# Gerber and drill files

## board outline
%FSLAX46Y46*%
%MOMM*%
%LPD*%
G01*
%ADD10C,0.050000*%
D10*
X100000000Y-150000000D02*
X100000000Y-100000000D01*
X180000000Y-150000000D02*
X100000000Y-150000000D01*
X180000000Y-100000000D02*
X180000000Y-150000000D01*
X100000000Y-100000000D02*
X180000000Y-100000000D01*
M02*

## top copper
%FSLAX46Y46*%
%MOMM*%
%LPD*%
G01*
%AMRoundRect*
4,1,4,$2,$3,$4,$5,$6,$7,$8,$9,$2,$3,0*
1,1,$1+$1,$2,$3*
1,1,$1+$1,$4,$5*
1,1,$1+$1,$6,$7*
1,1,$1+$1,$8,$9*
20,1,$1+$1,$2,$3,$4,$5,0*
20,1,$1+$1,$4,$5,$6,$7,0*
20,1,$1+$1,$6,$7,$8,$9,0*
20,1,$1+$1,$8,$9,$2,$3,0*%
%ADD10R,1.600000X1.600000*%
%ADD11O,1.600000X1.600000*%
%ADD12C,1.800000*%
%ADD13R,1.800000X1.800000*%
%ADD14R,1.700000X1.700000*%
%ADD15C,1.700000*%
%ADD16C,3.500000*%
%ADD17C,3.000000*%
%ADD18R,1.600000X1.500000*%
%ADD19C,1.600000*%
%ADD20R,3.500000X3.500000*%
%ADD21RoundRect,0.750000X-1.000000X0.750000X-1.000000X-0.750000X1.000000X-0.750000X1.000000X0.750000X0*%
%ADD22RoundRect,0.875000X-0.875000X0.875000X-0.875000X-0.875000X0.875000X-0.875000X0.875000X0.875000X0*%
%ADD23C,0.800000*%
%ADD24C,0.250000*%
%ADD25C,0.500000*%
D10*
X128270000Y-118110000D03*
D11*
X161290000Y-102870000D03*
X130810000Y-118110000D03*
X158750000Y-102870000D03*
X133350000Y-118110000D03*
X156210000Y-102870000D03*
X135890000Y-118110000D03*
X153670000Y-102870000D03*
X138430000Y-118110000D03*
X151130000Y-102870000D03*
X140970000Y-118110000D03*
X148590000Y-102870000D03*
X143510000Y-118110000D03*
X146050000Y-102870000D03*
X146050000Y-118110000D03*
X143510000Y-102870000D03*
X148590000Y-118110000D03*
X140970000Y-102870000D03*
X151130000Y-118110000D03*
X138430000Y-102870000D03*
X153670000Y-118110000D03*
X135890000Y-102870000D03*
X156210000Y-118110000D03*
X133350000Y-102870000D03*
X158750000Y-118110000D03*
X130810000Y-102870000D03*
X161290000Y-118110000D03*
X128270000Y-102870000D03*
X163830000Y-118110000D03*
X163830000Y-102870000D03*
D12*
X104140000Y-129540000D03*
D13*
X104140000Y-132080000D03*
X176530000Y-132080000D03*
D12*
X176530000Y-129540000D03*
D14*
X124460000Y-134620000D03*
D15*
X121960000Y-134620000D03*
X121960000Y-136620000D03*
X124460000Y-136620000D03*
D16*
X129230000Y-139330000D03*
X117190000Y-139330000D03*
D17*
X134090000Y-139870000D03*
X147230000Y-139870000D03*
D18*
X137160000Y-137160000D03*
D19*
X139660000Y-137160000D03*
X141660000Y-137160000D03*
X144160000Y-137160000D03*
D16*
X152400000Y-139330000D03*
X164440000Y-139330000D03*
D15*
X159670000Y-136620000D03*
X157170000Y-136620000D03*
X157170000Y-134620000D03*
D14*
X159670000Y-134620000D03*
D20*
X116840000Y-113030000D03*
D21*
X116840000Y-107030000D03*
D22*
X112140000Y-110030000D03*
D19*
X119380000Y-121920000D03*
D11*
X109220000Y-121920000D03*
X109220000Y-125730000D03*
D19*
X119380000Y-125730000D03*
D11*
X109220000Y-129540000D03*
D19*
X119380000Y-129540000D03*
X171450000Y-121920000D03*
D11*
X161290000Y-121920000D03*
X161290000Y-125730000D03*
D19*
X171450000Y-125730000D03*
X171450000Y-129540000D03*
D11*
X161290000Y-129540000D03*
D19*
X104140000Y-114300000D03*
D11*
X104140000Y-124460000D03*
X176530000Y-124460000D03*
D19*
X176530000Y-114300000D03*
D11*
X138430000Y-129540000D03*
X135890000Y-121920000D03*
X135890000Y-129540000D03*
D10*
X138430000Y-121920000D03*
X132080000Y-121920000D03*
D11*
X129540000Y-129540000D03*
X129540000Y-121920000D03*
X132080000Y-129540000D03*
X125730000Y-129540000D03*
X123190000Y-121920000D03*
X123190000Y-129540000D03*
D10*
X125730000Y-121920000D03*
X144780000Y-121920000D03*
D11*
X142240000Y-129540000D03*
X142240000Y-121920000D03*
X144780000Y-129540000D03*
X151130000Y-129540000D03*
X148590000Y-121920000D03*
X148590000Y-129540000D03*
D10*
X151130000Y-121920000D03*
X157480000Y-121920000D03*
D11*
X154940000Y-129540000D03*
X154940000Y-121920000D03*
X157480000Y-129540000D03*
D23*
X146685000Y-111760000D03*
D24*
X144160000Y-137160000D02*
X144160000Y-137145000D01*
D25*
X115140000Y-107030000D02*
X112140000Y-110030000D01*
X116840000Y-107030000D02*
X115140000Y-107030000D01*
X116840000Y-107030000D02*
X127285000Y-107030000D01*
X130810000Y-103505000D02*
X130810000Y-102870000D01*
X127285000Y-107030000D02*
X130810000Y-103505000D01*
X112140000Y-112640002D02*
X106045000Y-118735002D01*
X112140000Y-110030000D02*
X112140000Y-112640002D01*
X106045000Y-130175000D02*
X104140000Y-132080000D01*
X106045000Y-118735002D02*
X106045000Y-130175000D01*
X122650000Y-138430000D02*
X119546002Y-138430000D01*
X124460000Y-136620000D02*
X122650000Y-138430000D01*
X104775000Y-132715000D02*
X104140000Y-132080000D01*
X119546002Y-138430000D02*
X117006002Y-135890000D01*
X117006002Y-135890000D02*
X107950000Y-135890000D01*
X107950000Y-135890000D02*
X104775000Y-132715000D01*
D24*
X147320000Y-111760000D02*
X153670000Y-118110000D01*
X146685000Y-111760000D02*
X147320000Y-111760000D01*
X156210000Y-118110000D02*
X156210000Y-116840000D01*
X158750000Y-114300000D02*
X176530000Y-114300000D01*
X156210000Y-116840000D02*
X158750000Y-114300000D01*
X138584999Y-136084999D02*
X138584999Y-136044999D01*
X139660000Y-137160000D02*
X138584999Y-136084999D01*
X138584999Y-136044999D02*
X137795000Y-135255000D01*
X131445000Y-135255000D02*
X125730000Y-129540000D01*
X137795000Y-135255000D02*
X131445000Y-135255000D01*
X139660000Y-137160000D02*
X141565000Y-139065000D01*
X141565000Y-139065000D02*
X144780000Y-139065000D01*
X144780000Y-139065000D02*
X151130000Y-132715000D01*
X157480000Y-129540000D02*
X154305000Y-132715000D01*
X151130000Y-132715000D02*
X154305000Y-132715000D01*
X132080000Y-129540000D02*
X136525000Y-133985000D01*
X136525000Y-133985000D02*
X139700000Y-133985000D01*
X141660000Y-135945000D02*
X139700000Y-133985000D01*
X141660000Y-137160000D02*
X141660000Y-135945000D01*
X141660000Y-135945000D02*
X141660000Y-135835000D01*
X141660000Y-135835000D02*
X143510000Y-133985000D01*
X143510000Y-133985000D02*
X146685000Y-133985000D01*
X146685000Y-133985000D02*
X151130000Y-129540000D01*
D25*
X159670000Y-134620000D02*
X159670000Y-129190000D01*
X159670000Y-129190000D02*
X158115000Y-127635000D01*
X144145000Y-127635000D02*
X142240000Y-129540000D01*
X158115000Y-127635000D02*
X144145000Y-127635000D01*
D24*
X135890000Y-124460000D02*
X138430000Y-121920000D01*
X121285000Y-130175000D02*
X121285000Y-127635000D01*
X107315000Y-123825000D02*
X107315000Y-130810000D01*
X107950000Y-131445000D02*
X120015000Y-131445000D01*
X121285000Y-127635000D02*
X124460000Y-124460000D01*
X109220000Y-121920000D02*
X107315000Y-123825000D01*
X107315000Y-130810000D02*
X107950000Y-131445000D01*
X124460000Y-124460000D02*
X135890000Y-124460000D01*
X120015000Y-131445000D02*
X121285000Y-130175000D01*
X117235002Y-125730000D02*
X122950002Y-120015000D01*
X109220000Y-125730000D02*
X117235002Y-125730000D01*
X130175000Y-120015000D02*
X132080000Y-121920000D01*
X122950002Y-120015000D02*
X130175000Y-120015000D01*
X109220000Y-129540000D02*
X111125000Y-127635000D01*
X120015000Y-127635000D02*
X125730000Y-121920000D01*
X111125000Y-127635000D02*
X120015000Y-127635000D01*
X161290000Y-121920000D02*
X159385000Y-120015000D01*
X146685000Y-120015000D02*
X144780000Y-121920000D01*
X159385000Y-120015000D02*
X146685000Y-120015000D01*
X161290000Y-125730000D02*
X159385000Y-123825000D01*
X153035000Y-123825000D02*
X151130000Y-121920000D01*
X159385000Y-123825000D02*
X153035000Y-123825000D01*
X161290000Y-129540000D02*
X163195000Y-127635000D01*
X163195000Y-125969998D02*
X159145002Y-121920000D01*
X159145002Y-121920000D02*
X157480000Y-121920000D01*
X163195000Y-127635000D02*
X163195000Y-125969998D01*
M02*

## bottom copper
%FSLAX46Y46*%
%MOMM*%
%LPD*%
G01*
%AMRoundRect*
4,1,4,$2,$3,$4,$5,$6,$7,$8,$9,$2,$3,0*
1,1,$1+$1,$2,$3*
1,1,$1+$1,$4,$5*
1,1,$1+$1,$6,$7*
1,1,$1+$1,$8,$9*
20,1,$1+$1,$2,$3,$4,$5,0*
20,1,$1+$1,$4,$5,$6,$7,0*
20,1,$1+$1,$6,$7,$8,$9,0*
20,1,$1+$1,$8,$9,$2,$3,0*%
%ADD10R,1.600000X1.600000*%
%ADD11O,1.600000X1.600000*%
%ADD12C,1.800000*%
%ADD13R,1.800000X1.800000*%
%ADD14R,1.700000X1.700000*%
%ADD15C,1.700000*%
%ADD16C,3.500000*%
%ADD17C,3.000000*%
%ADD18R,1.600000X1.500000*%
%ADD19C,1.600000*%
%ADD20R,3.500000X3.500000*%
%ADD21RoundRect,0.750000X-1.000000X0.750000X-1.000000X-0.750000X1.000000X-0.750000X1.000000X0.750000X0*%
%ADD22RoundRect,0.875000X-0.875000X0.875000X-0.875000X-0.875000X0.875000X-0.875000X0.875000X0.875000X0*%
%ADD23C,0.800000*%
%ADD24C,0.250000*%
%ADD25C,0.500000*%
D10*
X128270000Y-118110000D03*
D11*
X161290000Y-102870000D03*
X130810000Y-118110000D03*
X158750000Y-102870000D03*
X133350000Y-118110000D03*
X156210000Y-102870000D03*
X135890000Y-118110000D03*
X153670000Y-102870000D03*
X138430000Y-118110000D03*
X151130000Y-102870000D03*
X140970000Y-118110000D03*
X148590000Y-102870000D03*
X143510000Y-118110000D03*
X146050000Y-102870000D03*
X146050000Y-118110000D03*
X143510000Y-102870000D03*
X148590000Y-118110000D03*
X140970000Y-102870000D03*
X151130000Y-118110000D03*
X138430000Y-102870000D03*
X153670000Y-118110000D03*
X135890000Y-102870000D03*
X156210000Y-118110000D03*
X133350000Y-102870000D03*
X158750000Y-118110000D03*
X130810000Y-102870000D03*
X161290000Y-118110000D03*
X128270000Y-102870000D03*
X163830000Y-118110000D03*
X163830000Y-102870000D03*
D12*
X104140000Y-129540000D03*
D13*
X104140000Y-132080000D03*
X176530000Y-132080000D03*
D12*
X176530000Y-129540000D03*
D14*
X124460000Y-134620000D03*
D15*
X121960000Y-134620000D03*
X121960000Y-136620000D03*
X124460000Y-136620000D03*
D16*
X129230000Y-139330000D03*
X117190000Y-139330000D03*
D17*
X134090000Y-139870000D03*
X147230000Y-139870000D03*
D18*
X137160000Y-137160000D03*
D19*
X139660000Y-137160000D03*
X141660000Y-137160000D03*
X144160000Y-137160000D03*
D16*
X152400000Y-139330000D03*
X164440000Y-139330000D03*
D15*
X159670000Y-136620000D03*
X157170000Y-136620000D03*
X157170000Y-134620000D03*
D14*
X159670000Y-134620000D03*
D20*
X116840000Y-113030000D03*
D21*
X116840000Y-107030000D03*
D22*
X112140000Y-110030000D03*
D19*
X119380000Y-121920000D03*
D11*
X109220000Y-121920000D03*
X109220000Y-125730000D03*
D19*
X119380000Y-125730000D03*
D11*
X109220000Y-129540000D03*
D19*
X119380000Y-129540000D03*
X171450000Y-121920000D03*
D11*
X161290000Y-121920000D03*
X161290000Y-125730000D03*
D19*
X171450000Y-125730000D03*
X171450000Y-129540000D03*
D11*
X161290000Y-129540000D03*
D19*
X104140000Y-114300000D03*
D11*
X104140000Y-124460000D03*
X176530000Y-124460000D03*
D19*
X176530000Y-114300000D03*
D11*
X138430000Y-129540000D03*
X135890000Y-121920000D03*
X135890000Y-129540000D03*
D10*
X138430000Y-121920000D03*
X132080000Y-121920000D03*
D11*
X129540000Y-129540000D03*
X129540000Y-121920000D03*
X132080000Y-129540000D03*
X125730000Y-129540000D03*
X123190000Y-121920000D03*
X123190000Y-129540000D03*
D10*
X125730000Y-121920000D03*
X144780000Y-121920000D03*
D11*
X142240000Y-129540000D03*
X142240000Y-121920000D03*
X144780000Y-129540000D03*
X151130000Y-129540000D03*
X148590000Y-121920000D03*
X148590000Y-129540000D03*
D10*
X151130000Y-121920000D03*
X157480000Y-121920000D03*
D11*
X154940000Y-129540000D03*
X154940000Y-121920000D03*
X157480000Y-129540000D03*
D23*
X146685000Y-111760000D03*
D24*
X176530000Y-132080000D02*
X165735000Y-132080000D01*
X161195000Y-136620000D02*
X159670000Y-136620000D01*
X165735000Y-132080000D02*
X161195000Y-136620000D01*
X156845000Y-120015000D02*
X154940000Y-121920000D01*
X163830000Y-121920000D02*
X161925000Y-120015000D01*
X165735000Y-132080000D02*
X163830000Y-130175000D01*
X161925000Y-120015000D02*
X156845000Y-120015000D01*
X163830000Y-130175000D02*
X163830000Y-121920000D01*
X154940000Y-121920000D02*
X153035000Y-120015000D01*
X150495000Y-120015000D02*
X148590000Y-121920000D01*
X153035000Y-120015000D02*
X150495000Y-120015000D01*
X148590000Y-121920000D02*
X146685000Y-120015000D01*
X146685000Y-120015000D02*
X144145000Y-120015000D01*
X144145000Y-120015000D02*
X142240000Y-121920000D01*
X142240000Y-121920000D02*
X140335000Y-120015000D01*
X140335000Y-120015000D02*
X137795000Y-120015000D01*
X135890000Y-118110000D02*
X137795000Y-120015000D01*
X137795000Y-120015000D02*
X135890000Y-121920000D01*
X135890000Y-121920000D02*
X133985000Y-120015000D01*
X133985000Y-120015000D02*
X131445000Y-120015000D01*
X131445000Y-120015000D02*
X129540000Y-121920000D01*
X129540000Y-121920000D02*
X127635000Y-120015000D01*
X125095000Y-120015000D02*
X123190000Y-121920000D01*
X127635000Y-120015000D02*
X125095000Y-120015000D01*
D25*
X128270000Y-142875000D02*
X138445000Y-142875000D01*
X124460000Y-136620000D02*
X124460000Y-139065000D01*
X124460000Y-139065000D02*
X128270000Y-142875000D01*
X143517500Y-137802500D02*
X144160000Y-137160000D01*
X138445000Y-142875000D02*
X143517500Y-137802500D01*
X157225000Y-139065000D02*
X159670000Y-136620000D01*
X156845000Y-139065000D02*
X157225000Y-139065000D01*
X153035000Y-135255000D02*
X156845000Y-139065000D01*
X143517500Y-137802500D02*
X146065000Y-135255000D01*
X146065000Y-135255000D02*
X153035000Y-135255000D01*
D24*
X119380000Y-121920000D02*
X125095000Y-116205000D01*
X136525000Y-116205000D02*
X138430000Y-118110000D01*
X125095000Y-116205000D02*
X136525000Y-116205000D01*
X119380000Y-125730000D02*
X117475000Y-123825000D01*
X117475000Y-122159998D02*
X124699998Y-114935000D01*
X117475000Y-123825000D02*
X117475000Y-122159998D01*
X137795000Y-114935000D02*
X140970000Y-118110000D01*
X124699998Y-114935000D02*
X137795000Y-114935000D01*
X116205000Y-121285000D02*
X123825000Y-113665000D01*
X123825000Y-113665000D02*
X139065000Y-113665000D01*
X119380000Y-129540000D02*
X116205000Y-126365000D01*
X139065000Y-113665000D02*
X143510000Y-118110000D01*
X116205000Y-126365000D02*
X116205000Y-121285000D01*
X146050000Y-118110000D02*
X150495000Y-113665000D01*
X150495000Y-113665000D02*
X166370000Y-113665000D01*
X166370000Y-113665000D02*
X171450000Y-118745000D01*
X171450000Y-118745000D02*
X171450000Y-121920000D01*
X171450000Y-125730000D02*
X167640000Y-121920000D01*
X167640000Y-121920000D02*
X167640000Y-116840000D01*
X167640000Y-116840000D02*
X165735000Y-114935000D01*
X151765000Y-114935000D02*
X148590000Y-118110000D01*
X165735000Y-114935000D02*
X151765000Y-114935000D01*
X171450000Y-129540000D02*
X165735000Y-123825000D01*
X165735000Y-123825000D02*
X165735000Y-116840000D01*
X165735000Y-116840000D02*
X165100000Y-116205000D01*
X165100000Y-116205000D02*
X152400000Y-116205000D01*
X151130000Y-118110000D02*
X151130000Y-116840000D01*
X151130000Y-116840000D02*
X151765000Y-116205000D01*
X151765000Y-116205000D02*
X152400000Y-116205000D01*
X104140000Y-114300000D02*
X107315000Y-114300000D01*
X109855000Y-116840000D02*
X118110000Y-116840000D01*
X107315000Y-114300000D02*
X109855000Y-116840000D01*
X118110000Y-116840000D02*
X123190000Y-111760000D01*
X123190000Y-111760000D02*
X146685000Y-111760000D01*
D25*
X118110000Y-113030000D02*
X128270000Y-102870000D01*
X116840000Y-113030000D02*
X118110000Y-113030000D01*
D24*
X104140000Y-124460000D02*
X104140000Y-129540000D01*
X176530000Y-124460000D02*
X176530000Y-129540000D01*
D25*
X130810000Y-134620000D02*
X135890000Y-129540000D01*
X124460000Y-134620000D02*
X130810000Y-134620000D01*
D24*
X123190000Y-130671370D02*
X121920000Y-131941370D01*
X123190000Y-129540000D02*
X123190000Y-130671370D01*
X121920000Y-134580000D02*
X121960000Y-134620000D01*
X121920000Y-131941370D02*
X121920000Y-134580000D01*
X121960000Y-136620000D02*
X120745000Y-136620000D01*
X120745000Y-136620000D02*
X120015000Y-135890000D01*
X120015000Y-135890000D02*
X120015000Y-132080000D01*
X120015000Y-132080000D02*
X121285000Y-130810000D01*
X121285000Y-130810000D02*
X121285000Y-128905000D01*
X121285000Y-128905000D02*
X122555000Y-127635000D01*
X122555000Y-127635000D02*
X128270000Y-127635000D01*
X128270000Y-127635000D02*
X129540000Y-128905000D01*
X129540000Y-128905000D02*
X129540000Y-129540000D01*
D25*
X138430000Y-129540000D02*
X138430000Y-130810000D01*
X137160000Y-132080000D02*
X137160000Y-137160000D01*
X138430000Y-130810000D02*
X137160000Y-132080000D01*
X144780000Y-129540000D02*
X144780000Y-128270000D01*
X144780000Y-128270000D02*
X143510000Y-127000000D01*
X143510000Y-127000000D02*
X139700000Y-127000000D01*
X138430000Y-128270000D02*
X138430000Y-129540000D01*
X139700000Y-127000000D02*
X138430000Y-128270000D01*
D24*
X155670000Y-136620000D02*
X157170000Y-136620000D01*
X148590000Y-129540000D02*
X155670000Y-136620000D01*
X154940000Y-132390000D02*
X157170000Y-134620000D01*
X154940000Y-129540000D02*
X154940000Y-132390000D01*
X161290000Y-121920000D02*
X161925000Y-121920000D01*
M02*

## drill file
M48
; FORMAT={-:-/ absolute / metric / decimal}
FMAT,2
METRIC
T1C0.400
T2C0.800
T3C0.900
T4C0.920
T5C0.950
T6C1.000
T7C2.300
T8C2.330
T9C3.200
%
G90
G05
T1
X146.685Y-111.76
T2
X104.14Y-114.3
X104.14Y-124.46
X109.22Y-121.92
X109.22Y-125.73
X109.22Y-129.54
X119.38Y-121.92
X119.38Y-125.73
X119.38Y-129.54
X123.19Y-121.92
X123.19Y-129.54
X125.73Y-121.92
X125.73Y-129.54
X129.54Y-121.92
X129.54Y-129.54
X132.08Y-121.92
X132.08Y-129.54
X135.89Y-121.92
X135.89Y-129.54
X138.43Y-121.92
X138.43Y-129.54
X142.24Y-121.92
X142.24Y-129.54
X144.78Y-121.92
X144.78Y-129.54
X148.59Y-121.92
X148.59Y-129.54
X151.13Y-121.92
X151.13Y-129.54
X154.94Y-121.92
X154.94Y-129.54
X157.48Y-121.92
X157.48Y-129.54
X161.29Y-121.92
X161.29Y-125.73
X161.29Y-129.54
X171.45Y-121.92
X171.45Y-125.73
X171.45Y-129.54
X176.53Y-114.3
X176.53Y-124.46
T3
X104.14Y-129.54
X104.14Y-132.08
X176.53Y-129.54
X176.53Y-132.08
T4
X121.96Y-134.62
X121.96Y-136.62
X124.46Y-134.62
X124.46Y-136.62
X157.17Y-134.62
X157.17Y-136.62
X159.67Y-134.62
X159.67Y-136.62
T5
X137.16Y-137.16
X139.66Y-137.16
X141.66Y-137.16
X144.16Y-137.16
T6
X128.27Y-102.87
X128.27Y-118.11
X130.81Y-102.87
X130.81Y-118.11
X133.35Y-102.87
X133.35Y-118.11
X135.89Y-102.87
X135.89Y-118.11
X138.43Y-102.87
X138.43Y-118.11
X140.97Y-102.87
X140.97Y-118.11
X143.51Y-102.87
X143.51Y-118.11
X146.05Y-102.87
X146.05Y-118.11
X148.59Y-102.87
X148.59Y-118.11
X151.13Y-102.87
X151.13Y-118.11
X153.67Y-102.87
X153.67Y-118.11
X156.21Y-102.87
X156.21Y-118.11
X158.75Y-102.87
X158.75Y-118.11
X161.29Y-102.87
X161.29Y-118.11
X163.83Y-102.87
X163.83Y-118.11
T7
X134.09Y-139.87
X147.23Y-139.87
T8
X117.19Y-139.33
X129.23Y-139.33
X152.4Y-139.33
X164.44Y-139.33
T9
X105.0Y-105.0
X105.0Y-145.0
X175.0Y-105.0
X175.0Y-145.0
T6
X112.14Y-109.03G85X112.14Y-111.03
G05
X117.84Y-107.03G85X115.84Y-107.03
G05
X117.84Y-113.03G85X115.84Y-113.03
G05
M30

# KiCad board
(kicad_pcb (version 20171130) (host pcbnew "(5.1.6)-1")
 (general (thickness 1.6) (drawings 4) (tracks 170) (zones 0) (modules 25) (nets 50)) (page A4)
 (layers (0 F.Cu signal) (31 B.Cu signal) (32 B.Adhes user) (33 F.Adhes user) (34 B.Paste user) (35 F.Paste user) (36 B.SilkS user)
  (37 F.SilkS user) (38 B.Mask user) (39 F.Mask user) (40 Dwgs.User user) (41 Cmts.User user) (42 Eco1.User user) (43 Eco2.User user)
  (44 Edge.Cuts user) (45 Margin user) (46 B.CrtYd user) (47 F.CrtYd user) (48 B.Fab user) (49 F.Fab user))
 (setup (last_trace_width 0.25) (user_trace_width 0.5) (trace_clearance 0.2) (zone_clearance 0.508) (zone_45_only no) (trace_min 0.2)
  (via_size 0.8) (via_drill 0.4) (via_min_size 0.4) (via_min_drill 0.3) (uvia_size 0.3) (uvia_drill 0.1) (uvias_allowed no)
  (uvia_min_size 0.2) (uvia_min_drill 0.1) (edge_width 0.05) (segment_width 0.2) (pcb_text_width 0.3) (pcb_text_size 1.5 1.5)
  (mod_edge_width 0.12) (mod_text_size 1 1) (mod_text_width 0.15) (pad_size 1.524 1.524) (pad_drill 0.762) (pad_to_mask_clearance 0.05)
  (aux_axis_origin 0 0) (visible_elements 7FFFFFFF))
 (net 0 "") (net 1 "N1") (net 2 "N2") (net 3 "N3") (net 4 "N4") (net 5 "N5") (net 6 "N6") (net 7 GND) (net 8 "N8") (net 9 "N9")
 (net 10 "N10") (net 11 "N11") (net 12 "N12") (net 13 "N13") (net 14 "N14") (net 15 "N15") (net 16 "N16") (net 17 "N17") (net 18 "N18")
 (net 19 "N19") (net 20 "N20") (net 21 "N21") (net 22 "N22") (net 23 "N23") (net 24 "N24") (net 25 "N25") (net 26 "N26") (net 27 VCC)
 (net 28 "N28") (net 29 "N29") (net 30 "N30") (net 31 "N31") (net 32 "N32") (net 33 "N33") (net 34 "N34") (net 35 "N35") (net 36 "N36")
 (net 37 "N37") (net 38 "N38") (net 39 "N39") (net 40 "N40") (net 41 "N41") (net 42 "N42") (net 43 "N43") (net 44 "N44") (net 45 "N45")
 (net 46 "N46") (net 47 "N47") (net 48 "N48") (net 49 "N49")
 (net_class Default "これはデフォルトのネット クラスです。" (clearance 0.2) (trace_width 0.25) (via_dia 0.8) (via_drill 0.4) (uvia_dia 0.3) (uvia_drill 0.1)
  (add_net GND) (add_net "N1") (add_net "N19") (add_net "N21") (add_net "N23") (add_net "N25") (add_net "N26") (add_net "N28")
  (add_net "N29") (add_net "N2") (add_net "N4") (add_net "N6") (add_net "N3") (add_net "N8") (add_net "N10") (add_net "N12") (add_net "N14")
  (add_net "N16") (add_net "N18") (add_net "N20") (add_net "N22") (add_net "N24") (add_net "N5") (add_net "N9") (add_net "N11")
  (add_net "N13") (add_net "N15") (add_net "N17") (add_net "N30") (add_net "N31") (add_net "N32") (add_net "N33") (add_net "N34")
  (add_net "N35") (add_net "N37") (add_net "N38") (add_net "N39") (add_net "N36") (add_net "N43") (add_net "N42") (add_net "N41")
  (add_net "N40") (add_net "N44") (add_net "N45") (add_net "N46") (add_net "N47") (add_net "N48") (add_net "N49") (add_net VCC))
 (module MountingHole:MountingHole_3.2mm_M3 (layer F.Cu) (at 175 145)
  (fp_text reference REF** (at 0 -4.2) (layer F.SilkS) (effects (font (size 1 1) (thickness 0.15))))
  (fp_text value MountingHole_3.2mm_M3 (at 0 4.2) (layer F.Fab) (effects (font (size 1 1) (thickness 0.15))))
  (pad 1 np_thru_hole circle (at 0 0) (size 3.2 3.2) (drill 3.2) (layers *.Cu *.Mask)))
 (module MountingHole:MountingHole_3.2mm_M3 (layer F.Cu) (at 105 145)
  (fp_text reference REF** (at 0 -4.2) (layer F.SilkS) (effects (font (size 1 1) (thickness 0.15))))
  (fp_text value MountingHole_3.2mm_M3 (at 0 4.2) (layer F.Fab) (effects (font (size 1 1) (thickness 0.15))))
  (pad 1 np_thru_hole circle (at 0 0) (size 3.2 3.2) (drill 3.2) (layers *.Cu *.Mask)))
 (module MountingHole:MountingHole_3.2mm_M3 (layer F.Cu) (at 175 105)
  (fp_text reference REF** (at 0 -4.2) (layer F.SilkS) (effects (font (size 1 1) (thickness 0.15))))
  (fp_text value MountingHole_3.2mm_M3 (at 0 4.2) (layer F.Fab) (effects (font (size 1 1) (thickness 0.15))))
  (pad 1 np_thru_hole circle (at 0 0) (size 3.2 3.2) (drill 3.2) (layers *.Cu *.Mask)))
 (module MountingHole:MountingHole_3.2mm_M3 (layer F.Cu) (at 105 105)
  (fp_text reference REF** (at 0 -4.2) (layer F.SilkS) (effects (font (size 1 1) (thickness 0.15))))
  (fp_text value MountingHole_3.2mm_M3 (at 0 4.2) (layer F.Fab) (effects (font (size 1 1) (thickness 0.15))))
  (pad 1 np_thru_hole circle (at 0 0) (size 3.2 3.2) (drill 3.2) (layers *.Cu *.Mask)))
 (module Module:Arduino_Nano (layer F.Cu) (at 128.27 118.11 90)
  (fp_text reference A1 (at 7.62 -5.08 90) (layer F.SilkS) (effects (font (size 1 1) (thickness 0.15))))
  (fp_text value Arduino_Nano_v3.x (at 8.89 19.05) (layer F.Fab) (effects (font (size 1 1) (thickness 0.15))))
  (pad 1 thru_hole rect (at 0 0 90) (size 1.6 1.6) (drill 1) (layers *.Cu *.Mask) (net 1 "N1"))
  (pad 17 thru_hole oval (at 15.24 33.02 90) (size 1.6 1.6) (drill 1) (layers *.Cu *.Mask) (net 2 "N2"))
  (pad 2 thru_hole oval (at 0 2.54 90) (size 1.6 1.6) (drill 1) (layers *.Cu *.Mask) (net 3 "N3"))
  (pad 18 thru_hole oval (at 15.24 30.48 90) (size 1.6 1.6) (drill 1) (layers *.Cu *.Mask) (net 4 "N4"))
  (pad 3 thru_hole oval (at 0 5.08 90) (size 1.6 1.6) (drill 1) (layers *.Cu *.Mask) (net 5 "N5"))
  (pad 19 thru_hole oval (at 15.24 27.94 90) (size 1.6 1.6) (drill 1) (layers *.Cu *.Mask) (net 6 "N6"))
  (pad 4 thru_hole oval (at 0 7.62 90) (size 1.6 1.6) (drill 1) (layers *.Cu *.Mask) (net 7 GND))
  (pad 20 thru_hole oval (at 15.24 25.4 90) (size 1.6 1.6) (drill 1) (layers *.Cu *.Mask) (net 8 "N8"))
  (pad 5 thru_hole oval (at 0 10.16 90) (size 1.6 1.6) (drill 1) (layers *.Cu *.Mask) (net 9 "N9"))
  (pad 21 thru_hole oval (at 15.24 22.86 90) (size 1.6 1.6) (drill 1) (layers *.Cu *.Mask) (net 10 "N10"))
  (pad 6 thru_hole oval (at 0 12.7 90) (size 1.6 1.6) (drill 1) (layers *.Cu *.Mask) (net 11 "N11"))
  (pad 22 thru_hole oval (at 15.24 20.32 90) (size 1.6 1.6) (drill 1) (layers *.Cu *.Mask) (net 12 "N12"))
  (pad 7 thru_hole oval (at 0 15.24 90) (size 1.6 1.6) (drill 1) (layers *.Cu *.Mask) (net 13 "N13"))
  (pad 23 thru_hole oval (at 15.24 17.78 90) (size 1.6 1.6) (drill 1) (layers *.Cu *.Mask) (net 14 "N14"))
  (pad 8 thru_hole oval (at 0 17.78 90) (size 1.6 1.6) (drill 1) (layers *.Cu *.Mask) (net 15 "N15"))
  (pad 24 thru_hole oval (at 15.24 15.24 90) (size 1.6 1.6) (drill 1) (layers *.Cu *.Mask) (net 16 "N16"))
  (pad 9 thru_hole oval (at 0 20.32 90) (size 1.6 1.6) (drill 1) (layers *.Cu *.Mask) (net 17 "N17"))
  (pad 25 thru_hole oval (at 15.24 12.7 90) (size 1.6 1.6) (drill 1) (layers *.Cu *.Mask) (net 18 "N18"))
  (pad 10 thru_hole oval (at 0 22.86 90) (size 1.6 1.6) (drill 1) (layers *.Cu *.Mask) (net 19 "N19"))
  (pad 26 thru_hole oval (at 15.24 10.16 90) (size 1.6 1.6) (drill 1) (layers *.Cu *.Mask) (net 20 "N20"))
  (pad 11 thru_hole oval (at 0 25.4 90) (size 1.6 1.6) (drill 1) (layers *.Cu *.Mask) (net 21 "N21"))
  (pad 27 thru_hole oval (at 15.24 7.62 90) (size 1.6 1.6) (drill 1) (layers *.Cu *.Mask) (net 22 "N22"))
  (pad 12 thru_hole oval (at 0 27.94 90) (size 1.6 1.6) (drill 1) (layers *.Cu *.Mask) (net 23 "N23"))
  (pad 28 thru_hole oval (at 15.24 5.08 90) (size 1.6 1.6) (drill 1) (layers *.Cu *.Mask) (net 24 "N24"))
  (pad 13 thru_hole oval (at 0 30.48 90) (size 1.6 1.6) (drill 1) (layers *.Cu *.Mask) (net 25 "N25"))
  (pad 29 thru_hole oval (at 15.24 2.54 90) (size 1.6 1.6) (drill 1) (layers *.Cu *.Mask) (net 7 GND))
  (pad 14 thru_hole oval (at 0 33.02 90) (size 1.6 1.6) (drill 1) (layers *.Cu *.Mask) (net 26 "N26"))
  (pad 30 thru_hole oval (at 15.24 0 90) (size 1.6 1.6) (drill 1) (layers *.Cu *.Mask) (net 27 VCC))
  (pad 15 thru_hole oval (at 0 35.56 90) (size 1.6 1.6) (drill 1) (layers *.Cu *.Mask) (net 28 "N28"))
  (pad 16 thru_hole oval (at 15.24 35.56 90) (size 1.6 1.6) (drill 1) (layers *.Cu *.Mask) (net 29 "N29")))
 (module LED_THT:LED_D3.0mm (layer F.Cu) (at 104.14 132.08 90)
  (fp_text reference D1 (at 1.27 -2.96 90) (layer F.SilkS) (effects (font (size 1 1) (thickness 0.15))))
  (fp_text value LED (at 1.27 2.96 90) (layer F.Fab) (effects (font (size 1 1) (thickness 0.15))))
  (pad 2 thru_hole circle (at 2.54 0 90) (size 1.8 1.8) (drill 0.9) (layers *.Cu *.Mask) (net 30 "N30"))
  (pad 1 thru_hole rect (at 0 0 90) (size 1.8 1.8) (drill 0.9) (layers *.Cu *.Mask) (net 7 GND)))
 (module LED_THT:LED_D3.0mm (layer F.Cu) (at 176.53 132.08 90)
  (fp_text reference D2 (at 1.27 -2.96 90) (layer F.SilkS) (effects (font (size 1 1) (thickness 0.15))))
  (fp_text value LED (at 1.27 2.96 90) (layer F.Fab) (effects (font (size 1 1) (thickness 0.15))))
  (pad 1 thru_hole rect (at 0 0 90) (size 1.8 1.8) (drill 0.9) (layers *.Cu *.Mask) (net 7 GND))
  (pad 2 thru_hole circle (at 2.54 0 90) (size 1.8 1.8) (drill 0.9) (layers *.Cu *.Mask) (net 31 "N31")))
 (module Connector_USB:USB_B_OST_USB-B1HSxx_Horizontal (layer F.Cu) (at 124.46 134.62 270)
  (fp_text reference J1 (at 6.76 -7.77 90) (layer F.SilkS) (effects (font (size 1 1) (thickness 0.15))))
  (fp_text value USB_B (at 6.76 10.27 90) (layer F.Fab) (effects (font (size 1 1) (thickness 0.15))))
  (pad 1 thru_hole rect (at 0 0 270) (size 1.7 1.7) (drill 0.92) (layers *.Cu *.Mask) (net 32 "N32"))
  (pad 2 thru_hole circle (at 0 2.5 270) (size 1.7 1.7) (drill 0.92) (layers *.Cu *.Mask) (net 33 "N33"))
  (pad 3 thru_hole circle (at 2 2.5 270) (size 1.7 1.7) (drill 0.92) (layers *.Cu *.Mask) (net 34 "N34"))
  (pad 4 thru_hole circle (at 2 0 270) (size 1.7 1.7) (drill 0.92) (layers *.Cu *.Mask) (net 7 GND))
  (pad 5 thru_hole circle (at 4.71 -4.77 270) (size 3.5 3.5) (drill 2.33) (layers *.Cu *.Mask) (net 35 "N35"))
  (pad 5 thru_hole circle (at 4.71 7.27 270) (size 3.5 3.5) (drill 2.33) (layers *.Cu *.Mask) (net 35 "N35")))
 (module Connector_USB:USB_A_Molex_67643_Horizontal (layer F.Cu) (at 137.16 137.16)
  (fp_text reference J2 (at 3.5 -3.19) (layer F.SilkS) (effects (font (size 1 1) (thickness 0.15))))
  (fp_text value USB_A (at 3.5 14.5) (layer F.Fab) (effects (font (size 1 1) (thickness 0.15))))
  (pad 5 thru_hole circle (at -3.07 2.71) (size 3 3) (drill 2.3) (layers *.Cu *.Mask) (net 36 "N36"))
  (pad 5 thru_hole circle (at 10.07 2.71) (size 3 3) (drill 2.3) (layers *.Cu *.Mask) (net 36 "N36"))
  (pad 1 thru_hole rect (at 0 0) (size 1.6 1.5) (drill 0.95) (layers *.Cu *.Mask) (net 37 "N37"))
  (pad 2 thru_hole circle (at 2.5 0) (size 1.6 1.6) (drill 0.95) (layers *.Cu *.Mask) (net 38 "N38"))
  (pad 3 thru_hole circle (at 4.5 0) (size 1.6 1.6) (drill 0.95) (layers *.Cu *.Mask) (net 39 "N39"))
  (pad 4 thru_hole circle (at 7 0) (size 1.6 1.6) (drill 0.95) (layers *.Cu *.Mask) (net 7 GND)))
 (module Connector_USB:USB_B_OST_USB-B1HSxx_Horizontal (layer F.Cu) (at 159.67 134.62 270)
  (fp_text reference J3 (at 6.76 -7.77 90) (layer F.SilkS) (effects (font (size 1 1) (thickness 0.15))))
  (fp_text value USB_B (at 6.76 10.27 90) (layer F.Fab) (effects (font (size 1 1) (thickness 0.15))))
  (pad 5 thru_hole circle (at 4.71 7.27 270) (size 3.5 3.5) (drill 2.33) (layers *.Cu *.Mask) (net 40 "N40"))
  (pad 5 thru_hole circle (at 4.71 -4.77 270) (size 3.5 3.5) (drill 2.33) (layers *.Cu *.Mask) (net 40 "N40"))
  (pad 4 thru_hole circle (at 2 0 270) (size 1.7 1.7) (drill 0.92) (layers *.Cu *.Mask) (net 7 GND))
  (pad 3 thru_hole circle (at 2 2.5 270) (size 1.7 1.7) (drill 0.92) (layers *.Cu *.Mask) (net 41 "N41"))
  (pad 2 thru_hole circle (at 0 2.5 270) (size 1.7 1.7) (drill 0.92) (layers *.Cu *.Mask) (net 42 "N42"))
  (pad 1 thru_hole rect (at 0 0 270) (size 1.7 1.7) (drill 0.92) (layers *.Cu *.Mask) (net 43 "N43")))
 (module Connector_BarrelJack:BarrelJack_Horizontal (layer F.Cu) (at 116.84 113.03 270)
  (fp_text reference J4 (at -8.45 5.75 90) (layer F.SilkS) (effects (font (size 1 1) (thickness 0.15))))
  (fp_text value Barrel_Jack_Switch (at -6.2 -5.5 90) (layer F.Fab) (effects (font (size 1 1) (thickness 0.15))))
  (pad 1 thru_hole rect (at 0 0 270) (size 3.5 3.5) (drill oval 1 3) (layers *.Cu *.Mask) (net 27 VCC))
  (pad 2 thru_hole roundrect (at -6 0 270) (size 3 3.5) (drill oval 1 3) (layers *.Cu *.Mask) (roundrect_rratio 0.25) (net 7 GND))
  (pad 3 thru_hole roundrect (at -3 4.7 270) (size 3.5 3.5) (drill oval 3 1) (layers *.Cu *.Mask) (roundrect_rratio 0.25) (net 7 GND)))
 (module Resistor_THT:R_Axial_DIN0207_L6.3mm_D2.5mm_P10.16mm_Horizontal (layer F.Cu) (at 119.38 121.92 180)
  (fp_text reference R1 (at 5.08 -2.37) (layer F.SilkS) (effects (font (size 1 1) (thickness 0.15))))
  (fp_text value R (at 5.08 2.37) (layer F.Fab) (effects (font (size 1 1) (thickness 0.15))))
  (pad 1 thru_hole circle (at 0 0 180) (size 1.6 1.6) (drill 0.8) (layers *.Cu *.Mask) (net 9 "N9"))
  (pad 2 thru_hole oval (at 10.16 0 180) (size 1.6 1.6) (drill 0.8) (layers *.Cu *.Mask) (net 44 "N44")))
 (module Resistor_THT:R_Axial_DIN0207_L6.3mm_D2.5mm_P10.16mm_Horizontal (layer F.Cu) (at 119.38 125.73 180)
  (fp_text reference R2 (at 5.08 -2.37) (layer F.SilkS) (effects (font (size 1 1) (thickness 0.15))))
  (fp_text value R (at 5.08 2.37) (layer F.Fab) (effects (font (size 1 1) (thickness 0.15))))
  (pad 2 thru_hole oval (at 10.16 0 180) (size 1.6 1.6) (drill 0.8) (layers *.Cu *.Mask) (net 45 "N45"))
  (pad 1 thru_hole circle (at 0 0 180) (size 1.6 1.6) (drill 0.8) (layers *.Cu *.Mask) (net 11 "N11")))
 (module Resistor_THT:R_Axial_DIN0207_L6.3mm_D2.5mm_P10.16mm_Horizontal (layer F.Cu) (at 119.38 129.54 180)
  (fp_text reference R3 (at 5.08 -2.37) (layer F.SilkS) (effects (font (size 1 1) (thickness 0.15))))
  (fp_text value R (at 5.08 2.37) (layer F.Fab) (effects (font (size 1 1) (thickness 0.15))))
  (pad 2 thru_hole oval (at 10.16 0 180) (size 1.6 1.6) (drill 0.8) (layers *.Cu *.Mask) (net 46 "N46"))
  (pad 1 thru_hole circle (at 0 0 180) (size 1.6 1.6) (drill 0.8) (layers *.Cu *.Mask) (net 13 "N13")))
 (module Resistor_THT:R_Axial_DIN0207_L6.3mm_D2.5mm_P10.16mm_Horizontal (layer F.Cu) (at 171.45 121.92 180)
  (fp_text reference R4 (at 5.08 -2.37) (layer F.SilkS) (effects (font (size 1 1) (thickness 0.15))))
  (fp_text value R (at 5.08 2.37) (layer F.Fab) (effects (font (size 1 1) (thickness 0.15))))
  (pad 1 thru_hole circle (at 0 0 180) (size 1.6 1.6) (drill 0.8) (layers *.Cu *.Mask) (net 15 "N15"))
  (pad 2 thru_hole oval (at 10.16 0 180) (size 1.6 1.6) (drill 0.8) (layers *.Cu *.Mask) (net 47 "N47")))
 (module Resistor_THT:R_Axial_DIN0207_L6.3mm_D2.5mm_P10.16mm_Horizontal (layer F.Cu) (at 171.45 125.73 180)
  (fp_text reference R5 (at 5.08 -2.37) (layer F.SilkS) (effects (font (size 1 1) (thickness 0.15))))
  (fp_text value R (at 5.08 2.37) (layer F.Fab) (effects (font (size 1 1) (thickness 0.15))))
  (pad 2 thru_hole oval (at 10.16 0 180) (size 1.6 1.6) (drill 0.8) (layers *.Cu *.Mask) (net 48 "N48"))
  (pad 1 thru_hole circle (at 0 0 180) (size 1.6 1.6) (drill 0.8) (layers *.Cu *.Mask) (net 17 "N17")))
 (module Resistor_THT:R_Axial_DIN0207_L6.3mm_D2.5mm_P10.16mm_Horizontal (layer F.Cu) (at 171.45 129.54 180)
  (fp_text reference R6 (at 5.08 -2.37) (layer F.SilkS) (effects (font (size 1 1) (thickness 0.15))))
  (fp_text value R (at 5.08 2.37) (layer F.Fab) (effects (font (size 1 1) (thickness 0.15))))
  (pad 1 thru_hole circle (at 0 0 180) (size 1.6 1.6) (drill 0.8) (layers *.Cu *.Mask) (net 19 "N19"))
  (pad 2 thru_hole oval (at 10.16 0 180) (size 1.6 1.6) (drill 0.8) (layers *.Cu *.Mask) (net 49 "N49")))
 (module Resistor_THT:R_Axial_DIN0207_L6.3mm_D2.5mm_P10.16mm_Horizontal (layer F.Cu) (at 104.14 114.3 270)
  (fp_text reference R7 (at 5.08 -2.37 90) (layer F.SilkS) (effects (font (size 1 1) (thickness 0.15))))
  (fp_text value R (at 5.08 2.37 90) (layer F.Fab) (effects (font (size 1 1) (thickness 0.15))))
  (pad 1 thru_hole circle (at 0 0 270) (size 1.6 1.6) (drill 0.8) (layers *.Cu *.Mask) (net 21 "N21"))
  (pad 2 thru_hole oval (at 10.16 0 270) (size 1.6 1.6) (drill 0.8) (layers *.Cu *.Mask) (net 30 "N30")))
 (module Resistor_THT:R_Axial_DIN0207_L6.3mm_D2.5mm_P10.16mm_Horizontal (layer F.Cu) (at 176.53 114.3 270)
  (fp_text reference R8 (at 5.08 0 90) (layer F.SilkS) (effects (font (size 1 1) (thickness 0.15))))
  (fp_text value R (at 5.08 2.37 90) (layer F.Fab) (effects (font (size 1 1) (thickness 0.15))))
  (pad 2 thru_hole oval (at 10.16 0 270) (size 1.6 1.6) (drill 0.8) (layers *.Cu *.Mask) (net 31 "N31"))
  (pad 1 thru_hole circle (at 0 0 270) (size 1.6 1.6) (drill 0.8) (layers *.Cu *.Mask) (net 23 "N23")))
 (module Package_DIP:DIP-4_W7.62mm (layer F.Cu) (at 138.43 121.92 270)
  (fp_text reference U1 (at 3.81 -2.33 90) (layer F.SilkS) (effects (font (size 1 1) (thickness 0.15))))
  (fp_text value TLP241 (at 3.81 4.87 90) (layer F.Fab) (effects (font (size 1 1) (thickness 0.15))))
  (pad 4 thru_hole oval (at 7.62 0 270) (size 1.6 1.6) (drill 0.8) (layers *.Cu *.Mask) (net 37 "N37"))
  (pad 2 thru_hole oval (at 0 2.54 270) (size 1.6 1.6) (drill 0.8) (layers *.Cu *.Mask) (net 7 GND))
  (pad 3 thru_hole oval (at 7.62 2.54 270) (size 1.6 1.6) (drill 0.8) (layers *.Cu *.Mask) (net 32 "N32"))
  (pad 1 thru_hole rect (at 0 0 270) (size 1.6 1.6) (drill 0.8) (layers *.Cu *.Mask) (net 44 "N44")))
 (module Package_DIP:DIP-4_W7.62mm (layer F.Cu) (at 132.08 121.92 270)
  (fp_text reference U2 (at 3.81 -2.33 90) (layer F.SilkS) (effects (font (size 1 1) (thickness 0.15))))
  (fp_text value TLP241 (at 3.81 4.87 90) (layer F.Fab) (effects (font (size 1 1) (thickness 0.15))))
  (pad 1 thru_hole rect (at 0 0 270) (size 1.6 1.6) (drill 0.8) (layers *.Cu *.Mask) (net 45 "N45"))
  (pad 3 thru_hole oval (at 7.62 2.54 270) (size 1.6 1.6) (drill 0.8) (layers *.Cu *.Mask) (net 34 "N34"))
  (pad 2 thru_hole oval (at 0 2.54 270) (size 1.6 1.6) (drill 0.8) (layers *.Cu *.Mask) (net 7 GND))
  (pad 4 thru_hole oval (at 7.62 0 270) (size 1.6 1.6) (drill 0.8) (layers *.Cu *.Mask) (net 39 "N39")))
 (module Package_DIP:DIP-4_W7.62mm (layer F.Cu) (at 125.73 121.92 270)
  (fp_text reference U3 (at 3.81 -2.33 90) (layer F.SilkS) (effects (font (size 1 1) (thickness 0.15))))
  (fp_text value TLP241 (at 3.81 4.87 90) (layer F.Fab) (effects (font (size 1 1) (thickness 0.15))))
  (pad 4 thru_hole oval (at 7.62 0 270) (size 1.6 1.6) (drill 0.8) (layers *.Cu *.Mask) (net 38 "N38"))
  (pad 2 thru_hole oval (at 0 2.54 270) (size 1.6 1.6) (drill 0.8) (layers *.Cu *.Mask) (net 7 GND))
  (pad 3 thru_hole oval (at 7.62 2.54 270) (size 1.6 1.6) (drill 0.8) (layers *.Cu *.Mask) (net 33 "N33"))
  (pad 1 thru_hole rect (at 0 0 270) (size 1.6 1.6) (drill 0.8) (layers *.Cu *.Mask) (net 46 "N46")))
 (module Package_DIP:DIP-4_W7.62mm (layer F.Cu) (at 144.78 121.92 270)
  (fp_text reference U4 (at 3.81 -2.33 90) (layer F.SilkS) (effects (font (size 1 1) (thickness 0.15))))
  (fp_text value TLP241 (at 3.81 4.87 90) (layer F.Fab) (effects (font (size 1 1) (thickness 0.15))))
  (pad 1 thru_hole rect (at 0 0 270) (size 1.6 1.6) (drill 0.8) (layers *.Cu *.Mask) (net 47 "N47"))
  (pad 3 thru_hole oval (at 7.62 2.54 270) (size 1.6 1.6) (drill 0.8) (layers *.Cu *.Mask) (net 43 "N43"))
  (pad 2 thru_hole oval (at 0 2.54 270) (size 1.6 1.6) (drill 0.8) (layers *.Cu *.Mask) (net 7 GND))
  (pad 4 thru_hole oval (at 7.62 0 270) (size 1.6 1.6) (drill 0.8) (layers *.Cu *.Mask) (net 37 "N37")))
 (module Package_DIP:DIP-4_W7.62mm (layer F.Cu) (at 151.13 121.92 270)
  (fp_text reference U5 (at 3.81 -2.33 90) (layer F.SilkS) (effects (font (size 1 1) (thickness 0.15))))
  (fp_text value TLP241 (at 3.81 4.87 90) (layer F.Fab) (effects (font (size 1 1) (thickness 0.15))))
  (pad 4 thru_hole oval (at 7.62 0 270) (size 1.6 1.6) (drill 0.8) (layers *.Cu *.Mask) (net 39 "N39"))
  (pad 2 thru_hole oval (at 0 2.54 270) (size 1.6 1.6) (drill 0.8) (layers *.Cu *.Mask) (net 7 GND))
  (pad 3 thru_hole oval (at 7.62 2.54 270) (size 1.6 1.6) (drill 0.8) (layers *.Cu *.Mask) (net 41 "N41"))
  (pad 1 thru_hole rect (at 0 0 270) (size 1.6 1.6) (drill 0.8) (layers *.Cu *.Mask) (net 48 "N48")))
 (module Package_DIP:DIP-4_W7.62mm (layer F.Cu) (at 157.48 121.92 270)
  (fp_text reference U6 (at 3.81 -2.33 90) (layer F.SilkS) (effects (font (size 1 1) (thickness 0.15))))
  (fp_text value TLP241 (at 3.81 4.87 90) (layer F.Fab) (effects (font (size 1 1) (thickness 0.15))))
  (pad 1 thru_hole rect (at 0 0 270) (size 1.6 1.6) (drill 0.8) (layers *.Cu *.Mask) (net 49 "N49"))
  (pad 3 thru_hole oval (at 7.62 2.54 270) (size 1.6 1.6) (drill 0.8) (layers *.Cu *.Mask) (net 42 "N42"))
  (pad 2 thru_hole oval (at 0 2.54 270) (size 1.6 1.6) (drill 0.8) (layers *.Cu *.Mask) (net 7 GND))
  (pad 4 thru_hole oval (at 7.62 0 270) (size 1.6 1.6) (drill 0.8) (layers *.Cu *.Mask) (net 38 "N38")))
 (gr_line (start 100 150) (end 100 100) (layer Edge.Cuts) (width 0.05))
 (gr_line (start 180 150) (end 100 150) (layer Edge.Cuts) (width 0.05))
 (gr_line (start 180 100) (end 180 150) (layer Edge.Cuts) (width 0.05))
 (gr_line (start 100 100) (end 180 100) (layer Edge.Cuts) (width 0.05))
 (segment (start 144.16 137.16) (end 144.16 137.145) (width 0.25) (layer F.Cu) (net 7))
 (segment (start 176.53 132.08) (end 165.735 132.08) (width 0.25) (layer B.Cu) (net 7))
 (segment (start 161.195 136.62) (end 159.67 136.62) (width 0.25) (layer B.Cu) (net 7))
 (segment (start 165.735 132.08) (end 161.195 136.62) (width 0.25) (layer B.Cu) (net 7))
 (segment (start 156.845 120.015) (end 154.94 121.92) (width 0.25) (layer B.Cu) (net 7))
 (segment (start 163.83 121.92) (end 161.925 120.015) (width 0.25) (layer B.Cu) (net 7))
 (segment (start 165.735 132.08) (end 163.83 130.175) (width 0.25) (layer B.Cu) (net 7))
 (segment (start 161.925 120.015) (end 156.845 120.015) (width 0.25) (layer B.Cu) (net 7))
 (segment (start 163.83 130.175) (end 163.83 121.92) (width 0.25) (layer B.Cu) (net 7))
 (segment (start 154.94 121.92) (end 153.035 120.015) (width 0.25) (layer B.Cu) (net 7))
 (segment (start 150.495 120.015) (end 148.59 121.92) (width 0.25) (layer B.Cu) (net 7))
 (segment (start 153.035 120.015) (end 150.495 120.015) (width 0.25) (layer B.Cu) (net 7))
 (segment (start 148.59 121.92) (end 146.685 120.015) (width 0.25) (layer B.Cu) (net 7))
 (segment (start 146.685 120.015) (end 144.145 120.015) (width 0.25) (layer B.Cu) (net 7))
 (segment (start 144.145 120.015) (end 142.24 121.92) (width 0.25) (layer B.Cu) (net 7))
 (segment (start 142.24 121.92) (end 140.335 120.015) (width 0.25) (layer B.Cu) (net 7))
 (segment (start 140.335 120.015) (end 137.795 120.015) (width 0.25) (layer B.Cu) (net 7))
 (segment (start 135.89 118.11) (end 137.795 120.015) (width 0.25) (layer B.Cu) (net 7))
 (segment (start 137.795 120.015) (end 135.89 121.92) (width 0.25) (layer B.Cu) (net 7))
 (segment (start 135.89 121.92) (end 133.985 120.015) (width 0.25) (layer B.Cu) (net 7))
 (segment (start 133.985 120.015) (end 131.445 120.015) (width 0.25) (layer B.Cu) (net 7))
 (segment (start 131.445 120.015) (end 129.54 121.92) (width 0.25) (layer B.Cu) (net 7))
 (segment (start 129.54 121.92) (end 127.635 120.015) (width 0.25) (layer B.Cu) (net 7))
 (segment (start 125.095 120.015) (end 123.19 121.92) (width 0.25) (layer B.Cu) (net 7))
 (segment (start 127.635 120.015) (end 125.095 120.015) (width 0.25) (layer B.Cu) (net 7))
 (segment (start 115.14 107.03) (end 112.14 110.03) (width 0.5) (layer F.Cu) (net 7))
 (segment (start 116.84 107.03) (end 115.14 107.03) (width 0.5) (layer F.Cu) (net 7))
 (segment (start 116.84 107.03) (end 127.285 107.03) (width 0.5) (layer F.Cu) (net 7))
 (segment (start 130.81 103.505) (end 130.81 102.87) (width 0.5) (layer F.Cu) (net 7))
 (segment (start 127.285 107.03) (end 130.81 103.505) (width 0.5) (layer F.Cu) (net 7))
 (segment (start 112.14 112.640002) (end 106.045 118.735002) (width 0.5) (layer F.Cu) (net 7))
 (segment (start 112.14 110.03) (end 112.14 112.640002) (width 0.5) (layer F.Cu) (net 7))
 (segment (start 106.045 130.175) (end 104.14 132.08) (width 0.5) (layer F.Cu) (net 7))
 (segment (start 106.045 118.735002) (end 106.045 130.175) (width 0.5) (layer F.Cu) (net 7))
 (segment (start 122.65 138.43) (end 119.546002 138.43) (width 0.5) (layer F.Cu) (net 7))
 (segment (start 124.46 136.62) (end 122.65 138.43) (width 0.5) (layer F.Cu) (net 7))
 (segment (start 104.775 132.715) (end 104.14 132.08) (width 0.5) (layer F.Cu) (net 7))
 (segment (start 119.546002 138.43) (end 117.006002 135.89) (width 0.5) (layer F.Cu) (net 7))
 (segment (start 117.006002 135.89) (end 107.95 135.89) (width 0.5) (layer F.Cu) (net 7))
 (segment (start 107.95 135.89) (end 104.775 132.715) (width 0.5) (layer F.Cu) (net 7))
 (segment (start 128.27 142.875) (end 138.445 142.875) (width 0.5) (layer B.Cu) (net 7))
 (segment (start 124.46 136.62) (end 124.46 139.065) (width 0.5) (layer B.Cu) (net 7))
 (segment (start 124.46 139.065) (end 128.27 142.875) (width 0.5) (layer B.Cu) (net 7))
 (segment (start 143.5175 137.8025) (end 144.16 137.16) (width 0.5) (layer B.Cu) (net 7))
 (segment (start 138.445 142.875) (end 143.5175 137.8025) (width 0.5) (layer B.Cu) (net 7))
 (segment (start 157.225 139.065) (end 159.67 136.62) (width 0.5) (layer B.Cu) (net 7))
 (segment (start 156.845 139.065) (end 157.225 139.065) (width 0.5) (layer B.Cu) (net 7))
 (segment (start 153.035 135.255) (end 156.845 139.065) (width 0.5) (layer B.Cu) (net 7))
 (segment (start 143.5175 137.8025) (end 146.065 135.255) (width 0.5) (layer B.Cu) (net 7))
 (segment (start 146.065 135.255) (end 153.035 135.255) (width 0.5) (layer B.Cu) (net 7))
 (segment (start 119.38 121.92) (end 125.095 116.205) (width 0.25) (layer B.Cu) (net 9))
 (segment (start 136.525 116.205) (end 138.43 118.11) (width 0.25) (layer B.Cu) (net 9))
 (segment (start 125.095 116.205) (end 136.525 116.205) (width 0.25) (layer B.Cu) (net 9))
 (segment (start 119.38 125.73) (end 117.475 123.825) (width 0.25) (layer B.Cu) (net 11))
 (segment (start 117.475 122.159998) (end 124.699998 114.935) (width 0.25) (layer B.Cu) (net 11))
 (segment (start 117.475 123.825) (end 117.475 122.159998) (width 0.25) (layer B.Cu) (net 11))
 (segment (start 137.795 114.935) (end 140.97 118.11) (width 0.25) (layer B.Cu) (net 11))
 (segment (start 124.699998 114.935) (end 137.795 114.935) (width 0.25) (layer B.Cu) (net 11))
 (segment (start 116.205 121.285) (end 123.825 113.665) (width 0.25) (layer B.Cu) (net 13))
 (segment (start 123.825 113.665) (end 139.065 113.665) (width 0.25) (layer B.Cu) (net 13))
 (segment (start 119.38 129.54) (end 116.205 126.365) (width 0.25) (layer B.Cu) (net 13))
 (segment (start 139.065 113.665) (end 143.51 118.11) (width 0.25) (layer B.Cu) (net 13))
 (segment (start 116.205 126.365) (end 116.205 121.285) (width 0.25) (layer B.Cu) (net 13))
 (segment (start 146.05 118.11) (end 150.495 113.665) (width 0.25) (layer B.Cu) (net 15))
 (segment (start 150.495 113.665) (end 166.37 113.665) (width 0.25) (layer B.Cu) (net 15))
 (segment (start 166.37 113.665) (end 171.45 118.745) (width 0.25) (layer B.Cu) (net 15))
 (segment (start 171.45 118.745) (end 171.45 121.92) (width 0.25) (layer B.Cu) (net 15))
 (segment (start 171.45 125.73) (end 167.64 121.92) (width 0.25) (layer B.Cu) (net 17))
 (segment (start 167.64 121.92) (end 167.64 116.84) (width 0.25) (layer B.Cu) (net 17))
 (segment (start 167.64 116.84) (end 165.735 114.935) (width 0.25) (layer B.Cu) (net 17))
 (segment (start 151.765 114.935) (end 148.59 118.11) (width 0.25) (layer B.Cu) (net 17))
 (segment (start 165.735 114.935) (end 151.765 114.935) (width 0.25) (layer B.Cu) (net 17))
 (segment (start 171.45 129.54) (end 165.735 123.825) (width 0.25) (layer B.Cu) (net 19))
 (segment (start 165.735 123.825) (end 165.735 116.84) (width 0.25) (layer B.Cu) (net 19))
 (segment (start 165.735 116.84) (end 165.1 116.205) (width 0.25) (layer B.Cu) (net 19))
 (segment (start 165.1 116.205) (end 152.4 116.205) (width 0.25) (layer B.Cu) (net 19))
 (segment (start 151.13 118.11) (end 151.13 116.84) (width 0.25) (layer B.Cu) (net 19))
 (segment (start 151.13 116.84) (end 151.765 116.205) (width 0.25) (layer B.Cu) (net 19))
 (segment (start 151.765 116.205) (end 152.4 116.205) (width 0.25) (layer B.Cu) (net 19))
 (segment (start 104.14 114.3) (end 107.315 114.3) (width 0.25) (layer B.Cu) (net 21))
 (segment (start 109.855 116.84) (end 118.11 116.84) (width 0.25) (layer B.Cu) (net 21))
 (segment (start 107.315 114.3) (end 109.855 116.84) (width 0.25) (layer B.Cu) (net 21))
 (via (at 146.685 111.76) (size 0.8) (drill 0.4) (layers F.Cu B.Cu) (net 21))
 (segment (start 118.11 116.84) (end 123.19 111.76) (width 0.25) (layer B.Cu) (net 21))
 (segment (start 123.19 111.76) (end 146.685 111.76) (width 0.25) (layer B.Cu) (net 21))
 (segment (start 147.32 111.76) (end 153.67 118.11) (width 0.25) (layer F.Cu) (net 21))
 (segment (start 146.685 111.76) (end 147.32 111.76) (width 0.25) (layer F.Cu) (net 21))
 (segment (start 156.21 118.11) (end 156.21 116.84) (width 0.25) (layer F.Cu) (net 23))
 (segment (start 158.75 114.3) (end 176.53 114.3) (width 0.25) (layer F.Cu) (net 23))
 (segment (start 156.21 116.84) (end 158.75 114.3) (width 0.25) (layer F.Cu) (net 23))
 (segment (start 118.11 113.03) (end 128.27 102.87) (width 0.5) (layer B.Cu) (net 27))
 (segment (start 116.84 113.03) (end 118.11 113.03) (width 0.5) (layer B.Cu) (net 27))
 (segment (start 104.14 124.46) (end 104.14 129.54) (width 0.25) (layer B.Cu) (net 30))
 (segment (start 176.53 124.46) (end 176.53 129.54) (width 0.25) (layer B.Cu) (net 31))
 (segment (start 130.81 134.62) (end 135.89 129.54) (width 0.5) (layer B.Cu) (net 32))
 (segment (start 124.46 134.62) (end 130.81 134.62) (width 0.5) (layer B.Cu) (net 32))
 (segment (start 123.19 130.67137) (end 121.92 131.94137) (width 0.25) (layer B.Cu) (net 33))
 (segment (start 123.19 129.54) (end 123.19 130.67137) (width 0.25) (layer B.Cu) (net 33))
 (segment (start 121.92 134.58) (end 121.96 134.62) (width 0.25) (layer B.Cu) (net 33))
 (segment (start 121.92 131.94137) (end 121.92 134.58) (width 0.25) (layer B.Cu) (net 33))
 (segment (start 121.96 136.62) (end 120.745 136.62) (width 0.25) (layer B.Cu) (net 34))
 (segment (start 120.745 136.62) (end 120.015 135.89) (width 0.25) (layer B.Cu) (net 34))
 (segment (start 120.015 135.89) (end 120.015 132.08) (width 0.25) (layer B.Cu) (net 34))
 (segment (start 120.015 132.08) (end 121.285 130.81) (width 0.25) (layer B.Cu) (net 34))
 (segment (start 121.285 130.81) (end 121.285 128.905) (width 0.25) (layer B.Cu) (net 34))
 (segment (start 121.285 128.905) (end 122.555 127.635) (width 0.25) (layer B.Cu) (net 34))
 (segment (start 122.555 127.635) (end 128.27 127.635) (width 0.25) (layer B.Cu) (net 34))
 (segment (start 128.27 127.635) (end 129.54 128.905) (width 0.25) (layer B.Cu) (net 34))
 (segment (start 129.54 128.905) (end 129.54 129.54) (width 0.25) (layer B.Cu) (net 34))
 (segment (start 138.43 129.54) (end 138.43 130.81) (width 0.5) (layer B.Cu) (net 37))
 (segment (start 137.16 132.08) (end 137.16 137.16) (width 0.5) (layer B.Cu) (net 37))
 (segment (start 138.43 130.81) (end 137.16 132.08) (width 0.5) (layer B.Cu) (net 37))
 (segment (start 144.78 129.54) (end 144.78 128.27) (width 0.5) (layer B.Cu) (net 37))
 (segment (start 144.78 128.27) (end 143.51 127) (width 0.5) (layer B.Cu) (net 37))
 (segment (start 143.51 127) (end 139.7 127) (width 0.5) (layer B.Cu) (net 37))
 (segment (start 138.43 128.27) (end 138.43 129.54) (width 0.5) (layer B.Cu) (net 37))
 (segment (start 139.7 127) (end 138.43 128.27) (width 0.5) (layer B.Cu) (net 37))
 (segment (start 138.584999 136.084999) (end 138.584999 136.044999) (width 0.25) (layer F.Cu) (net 38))
 (segment (start 139.66 137.16) (end 138.584999 136.084999) (width 0.25) (layer F.Cu) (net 38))
 (segment (start 138.584999 136.044999) (end 137.795 135.255) (width 0.25) (layer F.Cu) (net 38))
 (segment (start 131.445 135.255) (end 125.73 129.54) (width 0.25) (layer F.Cu) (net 38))
 (segment (start 137.795 135.255) (end 131.445 135.255) (width 0.25) (layer F.Cu) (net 38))
 (segment (start 139.66 137.16) (end 141.565 139.065) (width 0.25) (layer F.Cu) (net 38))
 (segment (start 141.565 139.065) (end 144.78 139.065) (width 0.25) (layer F.Cu) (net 38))
 (segment (start 144.78 139.065) (end 151.13 132.715) (width 0.25) (layer F.Cu) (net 38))
 (segment (start 157.48 129.54) (end 154.305 132.715) (width 0.25) (layer F.Cu) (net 38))
 (segment (start 151.13 132.715) (end 154.305 132.715) (width 0.25) (layer F.Cu) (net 38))
 (segment (start 132.08 129.54) (end 136.525 133.985) (width 0.25) (layer F.Cu) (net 39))
 (segment (start 136.525 133.985) (end 139.7 133.985) (width 0.25) (layer F.Cu) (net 39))
 (segment (start 141.66 135.945) (end 139.7 133.985) (width 0.25) (layer F.Cu) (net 39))
 (segment (start 141.66 137.16) (end 141.66 135.945) (width 0.25) (layer F.Cu) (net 39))
 (segment (start 141.66 135.945) (end 141.66 135.835) (width 0.25) (layer F.Cu) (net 39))
 (segment (start 141.66 135.835) (end 143.51 133.985) (width 0.25) (layer F.Cu) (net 39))
 (segment (start 143.51 133.985) (end 146.685 133.985) (width 0.25) (layer F.Cu) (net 39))
 (segment (start 146.685 133.985) (end 151.13 129.54) (width 0.25) (layer F.Cu) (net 39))
 (segment (start 155.67 136.62) (end 157.17 136.62) (width 0.25) (layer B.Cu) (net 41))
 (segment (start 148.59 129.54) (end 155.67 136.62) (width 0.25) (layer B.Cu) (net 41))
 (segment (start 154.94 132.39) (end 157.17 134.62) (width 0.25) (layer B.Cu) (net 42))
 (segment (start 154.94 129.54) (end 154.94 132.39) (width 0.25) (layer B.Cu) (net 42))
 (segment (start 159.67 134.62) (end 159.67 129.19) (width 0.5) (layer F.Cu) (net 43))
 (segment (start 159.67 129.19) (end 158.115 127.635) (width 0.5) (layer F.Cu) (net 43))
 (segment (start 144.145 127.635) (end 142.24 129.54) (width 0.5) (layer F.Cu) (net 43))
 (segment (start 158.115 127.635) (end 144.145 127.635) (width 0.5) (layer F.Cu) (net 43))
 (segment (start 135.89 124.46) (end 138.43 121.92) (width 0.25) (layer F.Cu) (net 44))
 (segment (start 121.285 130.175) (end 121.285 127.635) (width 0.25) (layer F.Cu) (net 44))
 (segment (start 107.315 123.825) (end 107.315 130.81) (width 0.25) (layer F.Cu) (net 44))
 (segment (start 107.95 131.445) (end 120.015 131.445) (width 0.25) (layer F.Cu) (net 44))
 (segment (start 121.285 127.635) (end 124.46 124.46) (width 0.25) (layer F.Cu) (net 44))
 (segment (start 109.22 121.92) (end 107.315 123.825) (width 0.25) (layer F.Cu) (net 44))
 (segment (start 107.315 130.81) (end 107.95 131.445) (width 0.25) (layer F.Cu) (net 44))
 (segment (start 124.46 124.46) (end 135.89 124.46) (width 0.25) (layer F.Cu) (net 44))
 (segment (start 120.015 131.445) (end 121.285 130.175) (width 0.25) (layer F.Cu) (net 44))
 (segment (start 117.235002 125.73) (end 122.950002 120.015) (width 0.25) (layer F.Cu) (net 45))
 (segment (start 109.22 125.73) (end 117.235002 125.73) (width 0.25) (layer F.Cu) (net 45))
 (segment (start 130.175 120.015) (end 132.08 121.92) (width 0.25) (layer F.Cu) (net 45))
 (segment (start 122.950002 120.015) (end 130.175 120.015) (width 0.25) (layer F.Cu) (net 45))
 (segment (start 109.22 129.54) (end 111.125 127.635) (width 0.25) (layer F.Cu) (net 46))
 (segment (start 120.015 127.635) (end 125.73 121.92) (width 0.25) (layer F.Cu) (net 46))
 (segment (start 111.125 127.635) (end 120.015 127.635) (width 0.25) (layer F.Cu) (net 46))
 (segment (start 161.29 121.92) (end 161.925 121.92) (width 0.25) (layer B.Cu) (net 47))
 (segment (start 161.29 121.92) (end 159.385 120.015) (width 0.25) (layer F.Cu) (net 47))
 (segment (start 146.685 120.015) (end 144.78 121.92) (width 0.25) (layer F.Cu) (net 47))
 (segment (start 159.385 120.015) (end 146.685 120.015) (width 0.25) (layer F.Cu) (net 47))
 (segment (start 161.29 125.73) (end 159.385 123.825) (width 0.25) (layer F.Cu) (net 48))
 (segment (start 153.035 123.825) (end 151.13 121.92) (width 0.25) (layer F.Cu) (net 48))
 (segment (start 159.385 123.825) (end 153.035 123.825) (width 0.25) (layer F.Cu) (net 48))
 (segment (start 161.29 129.54) (end 163.195 127.635) (width 0.25) (layer F.Cu) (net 49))
 (segment (start 163.195 125.969998) (end 159.145002 121.92) (width 0.25) (layer F.Cu) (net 49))
 (segment (start 159.145002 121.92) (end 157.48 121.92) (width 0.25) (layer F.Cu) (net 49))
 (segment (start 163.195 127.635) (end 163.195 125.969998) (width 0.25) (layer F.Cu) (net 49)))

